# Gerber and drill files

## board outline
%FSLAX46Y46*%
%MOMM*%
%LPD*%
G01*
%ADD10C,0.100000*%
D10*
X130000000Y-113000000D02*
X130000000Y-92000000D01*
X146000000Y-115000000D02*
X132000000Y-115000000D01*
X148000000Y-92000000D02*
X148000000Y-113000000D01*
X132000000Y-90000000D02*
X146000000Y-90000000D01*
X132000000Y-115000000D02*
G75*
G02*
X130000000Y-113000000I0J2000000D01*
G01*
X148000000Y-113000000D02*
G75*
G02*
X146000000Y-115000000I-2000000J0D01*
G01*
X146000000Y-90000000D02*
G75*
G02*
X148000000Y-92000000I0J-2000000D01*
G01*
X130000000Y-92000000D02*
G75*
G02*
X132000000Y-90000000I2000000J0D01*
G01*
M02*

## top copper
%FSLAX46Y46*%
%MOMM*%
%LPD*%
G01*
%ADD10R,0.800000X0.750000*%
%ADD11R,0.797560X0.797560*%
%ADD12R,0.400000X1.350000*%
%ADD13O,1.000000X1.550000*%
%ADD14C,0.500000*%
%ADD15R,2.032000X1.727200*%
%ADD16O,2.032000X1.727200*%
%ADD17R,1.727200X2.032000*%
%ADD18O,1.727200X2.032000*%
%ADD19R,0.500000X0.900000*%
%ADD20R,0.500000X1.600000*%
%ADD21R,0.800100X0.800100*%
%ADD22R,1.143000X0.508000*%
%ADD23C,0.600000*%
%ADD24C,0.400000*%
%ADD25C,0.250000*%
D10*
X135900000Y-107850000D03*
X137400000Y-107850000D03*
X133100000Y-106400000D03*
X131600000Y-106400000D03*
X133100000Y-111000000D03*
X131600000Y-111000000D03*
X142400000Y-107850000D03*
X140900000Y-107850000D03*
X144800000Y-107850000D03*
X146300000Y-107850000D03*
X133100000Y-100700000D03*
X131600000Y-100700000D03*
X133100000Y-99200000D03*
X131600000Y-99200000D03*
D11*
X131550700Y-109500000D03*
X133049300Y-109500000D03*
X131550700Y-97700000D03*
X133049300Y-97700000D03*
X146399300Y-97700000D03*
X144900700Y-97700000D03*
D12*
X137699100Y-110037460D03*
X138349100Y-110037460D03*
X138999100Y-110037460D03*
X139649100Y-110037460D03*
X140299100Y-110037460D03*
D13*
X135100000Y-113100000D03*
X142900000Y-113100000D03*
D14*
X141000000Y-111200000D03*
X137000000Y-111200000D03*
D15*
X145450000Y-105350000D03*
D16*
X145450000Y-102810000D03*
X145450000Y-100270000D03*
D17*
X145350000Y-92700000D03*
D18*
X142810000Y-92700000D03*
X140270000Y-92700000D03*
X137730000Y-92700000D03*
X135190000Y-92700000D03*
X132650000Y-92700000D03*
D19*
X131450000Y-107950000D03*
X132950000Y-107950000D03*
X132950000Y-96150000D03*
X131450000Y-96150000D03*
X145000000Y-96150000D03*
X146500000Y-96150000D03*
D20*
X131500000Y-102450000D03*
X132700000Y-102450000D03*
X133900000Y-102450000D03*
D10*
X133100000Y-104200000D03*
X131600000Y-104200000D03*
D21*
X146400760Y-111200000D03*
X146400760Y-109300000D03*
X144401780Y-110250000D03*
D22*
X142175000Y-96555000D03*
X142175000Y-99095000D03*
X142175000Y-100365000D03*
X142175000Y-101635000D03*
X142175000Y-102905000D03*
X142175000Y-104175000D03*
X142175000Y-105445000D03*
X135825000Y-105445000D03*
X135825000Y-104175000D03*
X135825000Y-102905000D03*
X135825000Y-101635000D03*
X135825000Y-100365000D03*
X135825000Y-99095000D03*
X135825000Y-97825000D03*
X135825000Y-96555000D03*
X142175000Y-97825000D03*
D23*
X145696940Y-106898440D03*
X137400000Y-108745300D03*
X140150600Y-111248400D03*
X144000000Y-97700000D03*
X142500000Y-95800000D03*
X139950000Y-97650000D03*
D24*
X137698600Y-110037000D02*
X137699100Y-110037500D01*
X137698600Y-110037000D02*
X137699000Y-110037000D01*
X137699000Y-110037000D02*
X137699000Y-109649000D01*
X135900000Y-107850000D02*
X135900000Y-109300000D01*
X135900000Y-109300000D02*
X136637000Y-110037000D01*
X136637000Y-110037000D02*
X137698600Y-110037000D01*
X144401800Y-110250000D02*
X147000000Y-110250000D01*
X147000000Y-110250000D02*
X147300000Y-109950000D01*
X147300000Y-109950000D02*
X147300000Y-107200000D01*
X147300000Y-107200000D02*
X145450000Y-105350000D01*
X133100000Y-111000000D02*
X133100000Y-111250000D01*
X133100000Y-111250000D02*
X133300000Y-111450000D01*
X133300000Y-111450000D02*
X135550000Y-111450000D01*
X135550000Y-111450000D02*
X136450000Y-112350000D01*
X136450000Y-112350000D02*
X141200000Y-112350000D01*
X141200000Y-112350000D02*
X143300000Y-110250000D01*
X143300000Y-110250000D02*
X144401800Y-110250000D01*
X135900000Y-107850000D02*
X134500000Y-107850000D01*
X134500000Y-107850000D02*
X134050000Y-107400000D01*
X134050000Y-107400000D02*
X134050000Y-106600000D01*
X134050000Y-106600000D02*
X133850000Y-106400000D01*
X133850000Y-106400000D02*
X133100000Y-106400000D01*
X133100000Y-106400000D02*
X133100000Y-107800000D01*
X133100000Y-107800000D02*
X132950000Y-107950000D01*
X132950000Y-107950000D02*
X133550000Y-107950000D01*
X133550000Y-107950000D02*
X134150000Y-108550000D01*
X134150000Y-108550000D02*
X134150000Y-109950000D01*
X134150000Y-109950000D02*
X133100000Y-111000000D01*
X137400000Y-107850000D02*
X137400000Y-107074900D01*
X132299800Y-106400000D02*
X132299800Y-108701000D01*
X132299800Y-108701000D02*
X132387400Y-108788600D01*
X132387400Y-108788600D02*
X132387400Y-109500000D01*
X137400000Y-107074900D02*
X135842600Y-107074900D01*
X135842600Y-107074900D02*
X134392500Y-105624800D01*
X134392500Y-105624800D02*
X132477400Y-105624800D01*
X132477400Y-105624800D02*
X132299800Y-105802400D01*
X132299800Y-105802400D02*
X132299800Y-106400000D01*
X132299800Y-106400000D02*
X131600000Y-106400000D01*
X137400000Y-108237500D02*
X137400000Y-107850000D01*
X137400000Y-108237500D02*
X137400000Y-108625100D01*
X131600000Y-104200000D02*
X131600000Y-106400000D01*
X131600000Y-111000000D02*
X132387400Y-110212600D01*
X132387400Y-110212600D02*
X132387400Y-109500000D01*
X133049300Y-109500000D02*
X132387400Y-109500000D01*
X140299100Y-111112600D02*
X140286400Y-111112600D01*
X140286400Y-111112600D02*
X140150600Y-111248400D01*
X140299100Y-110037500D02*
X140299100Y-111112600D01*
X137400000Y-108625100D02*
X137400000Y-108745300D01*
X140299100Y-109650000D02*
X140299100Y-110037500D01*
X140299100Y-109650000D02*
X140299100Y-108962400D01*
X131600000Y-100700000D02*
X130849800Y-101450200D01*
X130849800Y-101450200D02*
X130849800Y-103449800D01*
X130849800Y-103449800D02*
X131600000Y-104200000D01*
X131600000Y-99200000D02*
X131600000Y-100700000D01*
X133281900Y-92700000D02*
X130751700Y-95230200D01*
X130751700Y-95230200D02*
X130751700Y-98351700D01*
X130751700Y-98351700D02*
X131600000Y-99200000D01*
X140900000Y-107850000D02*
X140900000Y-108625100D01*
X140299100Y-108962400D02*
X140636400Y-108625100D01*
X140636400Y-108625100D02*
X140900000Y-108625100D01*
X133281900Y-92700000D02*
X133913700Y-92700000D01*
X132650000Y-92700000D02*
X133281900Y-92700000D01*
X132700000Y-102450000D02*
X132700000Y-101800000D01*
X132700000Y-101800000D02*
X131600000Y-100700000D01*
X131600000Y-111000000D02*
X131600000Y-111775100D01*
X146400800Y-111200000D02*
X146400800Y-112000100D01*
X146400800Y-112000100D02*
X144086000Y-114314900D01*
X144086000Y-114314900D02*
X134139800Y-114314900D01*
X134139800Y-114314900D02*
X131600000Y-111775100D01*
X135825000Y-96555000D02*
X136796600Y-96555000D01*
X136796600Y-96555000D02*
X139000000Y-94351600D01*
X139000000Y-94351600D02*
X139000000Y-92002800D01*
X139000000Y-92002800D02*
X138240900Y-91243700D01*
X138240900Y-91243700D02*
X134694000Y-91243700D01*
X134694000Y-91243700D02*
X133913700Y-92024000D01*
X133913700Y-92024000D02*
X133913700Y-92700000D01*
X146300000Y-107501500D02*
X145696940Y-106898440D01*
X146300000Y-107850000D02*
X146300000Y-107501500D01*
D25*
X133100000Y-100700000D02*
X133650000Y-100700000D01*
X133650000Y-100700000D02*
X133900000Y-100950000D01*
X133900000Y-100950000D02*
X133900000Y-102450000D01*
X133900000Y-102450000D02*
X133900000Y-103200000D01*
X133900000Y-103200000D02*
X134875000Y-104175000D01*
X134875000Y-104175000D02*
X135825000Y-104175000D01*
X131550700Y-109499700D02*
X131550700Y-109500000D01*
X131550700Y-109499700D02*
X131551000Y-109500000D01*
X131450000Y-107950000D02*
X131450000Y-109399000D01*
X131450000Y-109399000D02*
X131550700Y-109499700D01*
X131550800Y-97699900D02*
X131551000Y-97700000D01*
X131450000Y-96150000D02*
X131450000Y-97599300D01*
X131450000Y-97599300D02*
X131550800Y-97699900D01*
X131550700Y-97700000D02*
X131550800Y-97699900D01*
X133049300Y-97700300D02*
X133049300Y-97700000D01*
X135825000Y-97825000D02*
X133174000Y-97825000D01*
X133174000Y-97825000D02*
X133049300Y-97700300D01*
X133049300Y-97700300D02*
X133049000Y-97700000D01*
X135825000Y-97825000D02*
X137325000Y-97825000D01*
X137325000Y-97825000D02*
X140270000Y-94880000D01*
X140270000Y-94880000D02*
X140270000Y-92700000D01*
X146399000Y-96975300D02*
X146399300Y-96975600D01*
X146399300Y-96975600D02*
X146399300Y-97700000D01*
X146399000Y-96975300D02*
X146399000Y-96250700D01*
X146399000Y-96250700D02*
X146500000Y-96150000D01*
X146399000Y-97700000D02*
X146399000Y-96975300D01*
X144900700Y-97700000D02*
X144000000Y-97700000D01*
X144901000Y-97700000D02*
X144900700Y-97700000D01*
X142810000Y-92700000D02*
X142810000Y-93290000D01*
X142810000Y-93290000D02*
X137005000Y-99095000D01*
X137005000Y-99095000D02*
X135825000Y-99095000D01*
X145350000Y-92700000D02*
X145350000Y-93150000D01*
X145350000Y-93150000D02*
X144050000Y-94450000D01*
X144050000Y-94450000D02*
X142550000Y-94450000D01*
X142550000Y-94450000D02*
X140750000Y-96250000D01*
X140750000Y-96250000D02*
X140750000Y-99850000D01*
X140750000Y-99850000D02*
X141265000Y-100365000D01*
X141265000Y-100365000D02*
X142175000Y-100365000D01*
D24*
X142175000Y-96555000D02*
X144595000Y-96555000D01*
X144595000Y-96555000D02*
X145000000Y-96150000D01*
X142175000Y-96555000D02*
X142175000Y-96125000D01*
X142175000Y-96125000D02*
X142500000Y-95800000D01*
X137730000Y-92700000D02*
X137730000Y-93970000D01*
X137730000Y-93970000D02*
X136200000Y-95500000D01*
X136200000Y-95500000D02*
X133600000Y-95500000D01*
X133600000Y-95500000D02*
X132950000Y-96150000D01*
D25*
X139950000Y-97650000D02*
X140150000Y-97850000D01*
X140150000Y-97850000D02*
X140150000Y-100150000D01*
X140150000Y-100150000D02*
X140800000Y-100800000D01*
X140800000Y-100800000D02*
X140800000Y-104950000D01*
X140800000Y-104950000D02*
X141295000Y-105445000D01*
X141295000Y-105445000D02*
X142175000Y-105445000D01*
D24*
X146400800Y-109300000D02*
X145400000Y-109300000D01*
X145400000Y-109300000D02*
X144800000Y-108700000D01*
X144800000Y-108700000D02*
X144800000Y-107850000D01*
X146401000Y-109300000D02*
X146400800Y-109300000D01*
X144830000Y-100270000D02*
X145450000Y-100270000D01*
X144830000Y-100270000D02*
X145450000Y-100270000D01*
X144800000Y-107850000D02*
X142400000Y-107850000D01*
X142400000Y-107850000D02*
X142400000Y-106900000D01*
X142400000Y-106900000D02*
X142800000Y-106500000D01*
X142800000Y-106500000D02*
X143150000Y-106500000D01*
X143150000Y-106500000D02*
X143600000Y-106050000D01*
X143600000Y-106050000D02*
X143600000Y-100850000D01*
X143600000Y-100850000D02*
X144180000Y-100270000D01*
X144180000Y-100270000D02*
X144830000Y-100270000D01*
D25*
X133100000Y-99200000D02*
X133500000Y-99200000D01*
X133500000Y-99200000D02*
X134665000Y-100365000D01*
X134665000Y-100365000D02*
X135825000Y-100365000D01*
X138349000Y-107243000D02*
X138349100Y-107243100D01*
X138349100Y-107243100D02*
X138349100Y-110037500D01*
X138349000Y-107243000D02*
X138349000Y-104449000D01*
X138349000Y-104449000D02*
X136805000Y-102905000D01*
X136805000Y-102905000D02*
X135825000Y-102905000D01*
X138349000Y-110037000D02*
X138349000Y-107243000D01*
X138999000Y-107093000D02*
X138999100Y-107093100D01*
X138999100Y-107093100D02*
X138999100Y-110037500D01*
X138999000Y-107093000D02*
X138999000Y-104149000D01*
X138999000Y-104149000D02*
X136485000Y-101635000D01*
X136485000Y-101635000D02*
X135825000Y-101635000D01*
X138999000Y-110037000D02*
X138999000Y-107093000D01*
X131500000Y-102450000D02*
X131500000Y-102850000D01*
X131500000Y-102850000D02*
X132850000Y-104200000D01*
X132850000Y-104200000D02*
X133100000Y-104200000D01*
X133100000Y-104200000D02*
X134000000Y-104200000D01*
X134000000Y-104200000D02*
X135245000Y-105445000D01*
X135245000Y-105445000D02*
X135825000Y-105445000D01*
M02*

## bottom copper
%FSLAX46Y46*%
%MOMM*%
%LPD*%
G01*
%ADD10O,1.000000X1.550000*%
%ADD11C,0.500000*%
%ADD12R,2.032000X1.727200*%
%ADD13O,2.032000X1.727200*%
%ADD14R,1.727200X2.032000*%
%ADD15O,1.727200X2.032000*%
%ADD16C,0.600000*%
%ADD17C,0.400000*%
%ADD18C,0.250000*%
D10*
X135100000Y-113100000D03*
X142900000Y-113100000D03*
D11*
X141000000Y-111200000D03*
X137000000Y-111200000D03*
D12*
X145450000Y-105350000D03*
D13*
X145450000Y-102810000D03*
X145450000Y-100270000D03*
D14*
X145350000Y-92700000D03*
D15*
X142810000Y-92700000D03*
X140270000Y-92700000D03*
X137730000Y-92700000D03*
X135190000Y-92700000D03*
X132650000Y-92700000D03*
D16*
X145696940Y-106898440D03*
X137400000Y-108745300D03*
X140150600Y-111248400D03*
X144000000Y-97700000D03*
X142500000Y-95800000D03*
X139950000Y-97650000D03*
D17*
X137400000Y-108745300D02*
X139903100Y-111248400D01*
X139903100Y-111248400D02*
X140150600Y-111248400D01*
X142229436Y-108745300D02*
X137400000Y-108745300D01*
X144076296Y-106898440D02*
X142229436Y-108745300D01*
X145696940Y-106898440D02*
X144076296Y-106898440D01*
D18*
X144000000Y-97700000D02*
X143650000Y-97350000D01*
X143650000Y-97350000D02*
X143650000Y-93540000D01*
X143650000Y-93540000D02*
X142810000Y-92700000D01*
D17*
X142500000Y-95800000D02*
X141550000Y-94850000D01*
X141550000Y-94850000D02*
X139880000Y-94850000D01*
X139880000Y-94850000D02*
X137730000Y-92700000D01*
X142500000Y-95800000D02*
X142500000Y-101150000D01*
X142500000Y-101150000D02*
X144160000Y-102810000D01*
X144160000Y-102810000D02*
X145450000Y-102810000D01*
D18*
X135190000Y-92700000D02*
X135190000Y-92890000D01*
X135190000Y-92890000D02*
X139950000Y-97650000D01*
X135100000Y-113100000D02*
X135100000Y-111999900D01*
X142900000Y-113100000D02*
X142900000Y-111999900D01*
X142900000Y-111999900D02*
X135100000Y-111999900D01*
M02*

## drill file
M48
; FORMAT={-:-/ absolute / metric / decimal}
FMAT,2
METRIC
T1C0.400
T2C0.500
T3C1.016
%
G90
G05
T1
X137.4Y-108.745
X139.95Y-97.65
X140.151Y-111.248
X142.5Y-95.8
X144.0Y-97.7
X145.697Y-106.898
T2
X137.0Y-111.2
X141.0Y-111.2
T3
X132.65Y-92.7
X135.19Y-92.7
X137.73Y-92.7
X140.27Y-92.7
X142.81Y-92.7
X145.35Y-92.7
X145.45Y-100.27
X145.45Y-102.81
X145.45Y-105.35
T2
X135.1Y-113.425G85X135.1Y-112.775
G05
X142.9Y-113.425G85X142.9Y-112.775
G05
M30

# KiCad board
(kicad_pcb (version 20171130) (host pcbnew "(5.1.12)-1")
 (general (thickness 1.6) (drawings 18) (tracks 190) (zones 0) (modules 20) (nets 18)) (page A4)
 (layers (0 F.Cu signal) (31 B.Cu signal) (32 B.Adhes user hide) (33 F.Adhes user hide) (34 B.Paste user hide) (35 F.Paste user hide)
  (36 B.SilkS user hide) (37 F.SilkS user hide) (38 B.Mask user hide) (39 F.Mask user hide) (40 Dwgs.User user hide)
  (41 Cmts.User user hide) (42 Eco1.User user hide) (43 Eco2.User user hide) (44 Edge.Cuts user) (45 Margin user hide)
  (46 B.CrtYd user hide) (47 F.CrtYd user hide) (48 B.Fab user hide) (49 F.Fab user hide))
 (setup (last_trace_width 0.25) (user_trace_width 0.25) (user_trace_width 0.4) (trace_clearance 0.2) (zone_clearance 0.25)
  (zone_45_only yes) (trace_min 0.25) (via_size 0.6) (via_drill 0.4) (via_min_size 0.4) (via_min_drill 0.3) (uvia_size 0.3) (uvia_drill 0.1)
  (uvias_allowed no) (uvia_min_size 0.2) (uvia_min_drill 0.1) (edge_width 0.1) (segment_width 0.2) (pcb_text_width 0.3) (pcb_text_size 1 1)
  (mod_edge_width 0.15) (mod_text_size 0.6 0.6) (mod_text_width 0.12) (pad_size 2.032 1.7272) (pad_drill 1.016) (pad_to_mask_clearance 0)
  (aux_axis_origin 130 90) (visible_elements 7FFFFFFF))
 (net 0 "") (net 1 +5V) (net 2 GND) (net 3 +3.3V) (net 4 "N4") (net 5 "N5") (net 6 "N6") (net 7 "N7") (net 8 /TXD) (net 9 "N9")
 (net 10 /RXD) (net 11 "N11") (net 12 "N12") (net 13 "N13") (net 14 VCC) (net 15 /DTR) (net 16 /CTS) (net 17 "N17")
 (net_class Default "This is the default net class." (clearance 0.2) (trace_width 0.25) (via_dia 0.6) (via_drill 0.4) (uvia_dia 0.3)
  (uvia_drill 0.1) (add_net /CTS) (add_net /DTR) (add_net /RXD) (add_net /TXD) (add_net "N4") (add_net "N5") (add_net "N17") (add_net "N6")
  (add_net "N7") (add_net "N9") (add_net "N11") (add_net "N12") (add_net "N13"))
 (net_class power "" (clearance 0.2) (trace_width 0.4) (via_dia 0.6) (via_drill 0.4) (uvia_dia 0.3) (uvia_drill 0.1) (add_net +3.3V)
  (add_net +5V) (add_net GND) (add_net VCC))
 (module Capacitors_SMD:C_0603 (layer F.Cu) (at 136.65 107.85)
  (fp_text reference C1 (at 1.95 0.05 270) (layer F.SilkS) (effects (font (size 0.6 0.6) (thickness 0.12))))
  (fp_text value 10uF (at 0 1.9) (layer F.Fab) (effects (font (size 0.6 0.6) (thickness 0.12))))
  (pad 1 smd rect (at -0.75 0) (size 0.8 0.75) (layers F.Cu F.Paste F.Mask) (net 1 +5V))
  (pad 2 smd rect (at 0.75 0) (size 0.8 0.75) (layers F.Cu F.Paste F.Mask) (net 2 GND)))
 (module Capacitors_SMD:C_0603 (layer F.Cu) (at 132.35 106.4 180)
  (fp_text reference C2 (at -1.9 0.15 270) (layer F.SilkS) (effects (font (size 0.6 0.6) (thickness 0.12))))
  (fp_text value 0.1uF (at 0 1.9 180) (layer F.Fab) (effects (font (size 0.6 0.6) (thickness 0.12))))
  (pad 1 smd rect (at -0.75 0 180) (size 0.8 0.75) (layers F.Cu F.Paste F.Mask) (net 1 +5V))
  (pad 2 smd rect (at 0.75 0 180) (size 0.8 0.75) (layers F.Cu F.Paste F.Mask) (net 2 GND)))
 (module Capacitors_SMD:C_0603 (layer F.Cu) (at 132.35 111 180)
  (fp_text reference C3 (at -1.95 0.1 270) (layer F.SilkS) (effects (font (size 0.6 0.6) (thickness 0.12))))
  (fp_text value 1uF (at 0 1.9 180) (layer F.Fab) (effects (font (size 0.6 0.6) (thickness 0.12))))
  (pad 1 smd rect (at -0.75 0 180) (size 0.8 0.75) (layers F.Cu F.Paste F.Mask) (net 1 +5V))
  (pad 2 smd rect (at 0.75 0 180) (size 0.8 0.75) (layers F.Cu F.Paste F.Mask) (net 2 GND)))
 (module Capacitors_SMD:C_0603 (layer F.Cu) (at 141.65 107.85 180)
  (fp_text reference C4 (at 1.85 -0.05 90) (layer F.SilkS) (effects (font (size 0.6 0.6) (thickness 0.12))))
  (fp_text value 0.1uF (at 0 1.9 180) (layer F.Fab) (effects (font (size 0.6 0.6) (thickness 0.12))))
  (pad 1 smd rect (at -0.75 0 180) (size 0.8 0.75) (layers F.Cu F.Paste F.Mask) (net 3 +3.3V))
  (pad 2 smd rect (at 0.75 0 180) (size 0.8 0.75) (layers F.Cu F.Paste F.Mask) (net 2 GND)))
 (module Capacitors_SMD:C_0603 (layer F.Cu) (at 145.55 107.85)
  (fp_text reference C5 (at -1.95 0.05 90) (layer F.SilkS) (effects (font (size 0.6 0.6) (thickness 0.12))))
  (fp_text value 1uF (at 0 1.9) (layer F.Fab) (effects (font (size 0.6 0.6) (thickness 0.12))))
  (pad 1 smd rect (at -0.75 0) (size 0.8 0.75) (layers F.Cu F.Paste F.Mask) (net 3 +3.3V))
  (pad 2 smd rect (at 0.75 0) (size 0.8 0.75) (layers F.Cu F.Paste F.Mask) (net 2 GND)))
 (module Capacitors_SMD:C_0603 (layer F.Cu) (at 132.35 100.7 180)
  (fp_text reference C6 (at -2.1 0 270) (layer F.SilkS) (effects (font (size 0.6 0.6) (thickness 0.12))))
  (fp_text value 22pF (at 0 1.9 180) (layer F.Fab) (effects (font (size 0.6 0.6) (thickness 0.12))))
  (pad 1 smd rect (at -0.75 0 180) (size 0.8 0.75) (layers F.Cu F.Paste F.Mask) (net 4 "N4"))
  (pad 2 smd rect (at 0.75 0 180) (size 0.8 0.75) (layers F.Cu F.Paste F.Mask) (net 2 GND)))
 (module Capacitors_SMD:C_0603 (layer F.Cu) (at 132.35 99.2 180)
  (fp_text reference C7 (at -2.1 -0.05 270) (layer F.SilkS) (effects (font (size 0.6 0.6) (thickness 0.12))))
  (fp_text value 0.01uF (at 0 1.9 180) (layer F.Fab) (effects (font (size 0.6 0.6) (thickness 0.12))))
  (pad 1 smd rect (at -0.75 0 180) (size 0.8 0.75) (layers F.Cu F.Paste F.Mask) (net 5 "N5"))
  (pad 2 smd rect (at 0.75 0 180) (size 0.8 0.75) (layers F.Cu F.Paste F.Mask) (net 2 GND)))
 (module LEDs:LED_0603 (layer F.Cu) (at 132.3 109.5 180)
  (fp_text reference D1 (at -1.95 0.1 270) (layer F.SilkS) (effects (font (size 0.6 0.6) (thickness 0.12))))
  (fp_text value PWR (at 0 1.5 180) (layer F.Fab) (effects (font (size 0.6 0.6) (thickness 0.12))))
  (pad 2 smd rect (at 0.7493 0) (size 0.79756 0.79756) (layers F.Cu F.Paste F.Mask) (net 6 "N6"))
  (pad 1 smd rect (at -0.7493 0) (size 0.79756 0.79756) (layers F.Cu F.Paste F.Mask) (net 2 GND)))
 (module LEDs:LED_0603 (layer F.Cu) (at 132.3 97.7 180)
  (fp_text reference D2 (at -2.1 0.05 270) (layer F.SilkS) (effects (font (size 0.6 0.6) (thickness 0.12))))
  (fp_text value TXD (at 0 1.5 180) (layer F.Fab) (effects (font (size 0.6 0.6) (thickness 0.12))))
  (pad 2 smd rect (at 0.7493 0) (size 0.79756 0.79756) (layers F.Cu F.Paste F.Mask) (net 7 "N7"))
  (pad 1 smd rect (at -0.7493 0) (size 0.79756 0.79756) (layers F.Cu F.Paste F.Mask) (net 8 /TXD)))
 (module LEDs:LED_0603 (layer F.Cu) (at 145.65 97.7)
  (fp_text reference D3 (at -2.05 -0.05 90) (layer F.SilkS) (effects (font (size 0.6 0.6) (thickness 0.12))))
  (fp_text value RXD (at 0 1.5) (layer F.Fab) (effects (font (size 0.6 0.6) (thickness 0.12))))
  (pad 2 smd rect (at 0.7493 0 180) (size 0.79756 0.79756) (layers F.Cu F.Paste F.Mask) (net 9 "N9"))
  (pad 1 smd rect (at -0.7493 0 180) (size 0.79756 0.79756) (layers F.Cu F.Paste F.Mask) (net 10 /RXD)))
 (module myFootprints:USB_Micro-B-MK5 (layer F.Cu) (at 139 111.6)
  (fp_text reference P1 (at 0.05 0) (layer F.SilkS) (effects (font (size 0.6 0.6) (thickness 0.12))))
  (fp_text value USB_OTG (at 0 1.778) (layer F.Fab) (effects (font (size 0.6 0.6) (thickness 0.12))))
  (pad 1 smd rect (at -1.3009 -1.56254 90) (size 1.35 0.4) (layers F.Cu F.Paste F.Mask) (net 1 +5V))
  (pad 2 smd rect (at -0.6509 -1.56254 90) (size 1.35 0.4) (layers F.Cu F.Paste F.Mask) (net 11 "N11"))
  (pad 3 smd rect (at -0.0009 -1.56254 90) (size 1.35 0.4) (layers F.Cu F.Paste F.Mask) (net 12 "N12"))
  (pad 4 smd rect (at 0.6491 -1.56254 90) (size 1.35 0.4) (layers F.Cu F.Paste F.Mask))
  (pad 5 smd rect (at 1.2991 -1.56254 90) (size 1.35 0.4) (layers F.Cu F.Paste F.Mask) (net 2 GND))
  (pad 6 thru_hole oval (at -3.9 1.5 90) (size 1.55 1) (drill oval 1.15 0.5) (layers *.Cu *.Mask F.SilkS) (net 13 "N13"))
  (pad 6 thru_hole oval (at 3.9 1.5 90) (size 1.55 1) (drill oval 1.15 0.5) (layers *.Cu *.Mask F.SilkS) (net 13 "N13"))
  (pad "" thru_hole circle (at 2 -0.4) (size 0.5 0.5) (drill 0.5) (layers *.Cu *.Mask F.SilkS) (zone_connect 0))
  (pad "" thru_hole circle (at -2 -0.4) (size 0.5 0.5) (drill 0.5) (layers *.Cu *.Mask F.SilkS) (zone_connect 0)))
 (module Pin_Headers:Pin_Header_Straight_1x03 (layer F.Cu) (at 145.45 105.35 180)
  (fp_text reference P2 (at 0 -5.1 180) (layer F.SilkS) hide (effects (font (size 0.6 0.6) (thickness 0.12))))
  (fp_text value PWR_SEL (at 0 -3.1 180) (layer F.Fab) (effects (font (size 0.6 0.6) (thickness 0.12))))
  (pad 1 thru_hole rect (at 0 0 180) (size 2.032 1.7272) (drill 1.016) (layers *.Cu *.Mask F.SilkS) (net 1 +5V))
  (pad 2 thru_hole oval (at 0 2.54 180) (size 2.032 1.7272) (drill 1.016) (layers *.Cu *.Mask F.SilkS) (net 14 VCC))
  (pad 3 thru_hole oval (at 0 5.08 180) (size 2.032 1.7272) (drill 1.016) (layers *.Cu *.Mask F.SilkS) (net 3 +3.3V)))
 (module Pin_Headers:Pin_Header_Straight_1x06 (layer F.Cu) (at 145.35 92.7 270)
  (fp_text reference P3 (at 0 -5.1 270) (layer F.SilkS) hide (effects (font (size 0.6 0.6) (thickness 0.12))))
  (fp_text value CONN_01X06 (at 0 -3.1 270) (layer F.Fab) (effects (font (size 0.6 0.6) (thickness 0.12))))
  (pad 1 thru_hole rect (at 0 0 270) (size 2.032 1.7272) (drill 1.016) (layers *.Cu *.Mask F.SilkS) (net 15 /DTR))
  (pad 2 thru_hole oval (at 0 2.54 270) (size 2.032 1.7272) (drill 1.016) (layers *.Cu *.Mask F.SilkS) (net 10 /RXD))
  (pad 3 thru_hole oval (at 0 5.08 270) (size 2.032 1.7272) (drill 1.016) (layers *.Cu *.Mask F.SilkS) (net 8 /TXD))
  (pad 4 thru_hole oval (at 0 7.62 270) (size 2.032 1.7272) (drill 1.016) (layers *.Cu *.Mask F.SilkS) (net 14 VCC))
  (pad 5 thru_hole oval (at 0 10.16 270) (size 2.032 1.7272) (drill 1.016) (layers *.Cu *.Mask F.SilkS) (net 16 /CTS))
  (pad 6 thru_hole oval (at 0 12.7 270) (size 2.032 1.7272) (drill 1.016) (layers *.Cu *.Mask F.SilkS) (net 2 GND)))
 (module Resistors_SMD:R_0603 (layer F.Cu) (at 132.2 107.95)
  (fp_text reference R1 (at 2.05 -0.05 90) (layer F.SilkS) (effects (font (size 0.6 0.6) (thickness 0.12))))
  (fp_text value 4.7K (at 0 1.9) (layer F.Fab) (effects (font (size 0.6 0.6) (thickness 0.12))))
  (pad 1 smd rect (at -0.75 0) (size 0.5 0.9) (layers F.Cu F.Paste F.Mask) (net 6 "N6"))
  (pad 2 smd rect (at 0.75 0) (size 0.5 0.9) (layers F.Cu F.Paste F.Mask) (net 1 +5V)))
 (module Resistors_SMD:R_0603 (layer F.Cu) (at 132.2 96.15 180)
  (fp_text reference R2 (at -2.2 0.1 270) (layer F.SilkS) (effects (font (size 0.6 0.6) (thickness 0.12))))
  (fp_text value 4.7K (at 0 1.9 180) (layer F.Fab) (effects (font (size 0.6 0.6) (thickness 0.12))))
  (pad 1 smd rect (at -0.75 0 180) (size 0.5 0.9) (layers F.Cu F.Paste F.Mask) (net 14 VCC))
  (pad 2 smd rect (at 0.75 0 180) (size 0.5 0.9) (layers F.Cu F.Paste F.Mask) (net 7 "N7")))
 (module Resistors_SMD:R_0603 (layer F.Cu) (at 145.75 96.15)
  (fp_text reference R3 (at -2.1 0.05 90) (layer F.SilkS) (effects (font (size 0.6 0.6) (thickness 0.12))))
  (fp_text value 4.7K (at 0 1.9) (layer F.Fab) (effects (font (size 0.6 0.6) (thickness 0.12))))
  (pad 1 smd rect (at -0.75 0) (size 0.5 0.9) (layers F.Cu F.Paste F.Mask) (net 14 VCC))
  (pad 2 smd rect (at 0.75 0) (size 0.5 0.9) (layers F.Cu F.Paste F.Mask) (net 9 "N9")))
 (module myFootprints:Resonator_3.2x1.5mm (layer F.Cu) (at 132.7 102.45 180)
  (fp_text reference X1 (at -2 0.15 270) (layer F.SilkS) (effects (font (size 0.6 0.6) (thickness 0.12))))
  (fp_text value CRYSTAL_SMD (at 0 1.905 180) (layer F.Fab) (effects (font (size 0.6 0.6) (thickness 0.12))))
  (pad 2 smd rect (at 1.2 0 180) (size 0.5 1.6) (layers F.Cu F.Paste F.Mask) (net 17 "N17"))
  (pad 3 smd rect (at 0 0 180) (size 0.5 1.6) (layers F.Cu F.Paste F.Mask) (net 2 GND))
  (pad 1 smd rect (at -1.2 0 180) (size 0.5 1.6) (layers F.Cu F.Paste F.Mask) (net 4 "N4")))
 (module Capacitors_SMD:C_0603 (layer F.Cu) (at 132.35 104.2 180)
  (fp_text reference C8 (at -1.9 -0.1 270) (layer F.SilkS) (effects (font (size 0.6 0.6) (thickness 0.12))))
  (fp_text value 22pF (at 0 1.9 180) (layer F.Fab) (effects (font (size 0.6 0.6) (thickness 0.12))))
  (pad 1 smd rect (at -0.75 0 180) (size 0.8 0.75) (layers F.Cu F.Paste F.Mask) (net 17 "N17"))
  (pad 2 smd rect (at 0.75 0 180) (size 0.8 0.75) (layers F.Cu F.Paste F.Mask) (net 2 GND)))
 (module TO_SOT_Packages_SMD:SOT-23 (layer F.Cu) (at 145.4 110.25 90)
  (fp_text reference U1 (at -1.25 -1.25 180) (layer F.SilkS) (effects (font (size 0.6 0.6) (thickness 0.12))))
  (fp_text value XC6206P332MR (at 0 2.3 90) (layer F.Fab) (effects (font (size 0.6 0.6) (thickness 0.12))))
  (pad 1 smd rect (at -0.95 1.00076 90) (size 0.8001 0.8001) (layers F.Cu F.Paste F.Mask) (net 2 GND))
  (pad 2 smd rect (at 0.95 1.00076 90) (size 0.8001 0.8001) (layers F.Cu F.Paste F.Mask) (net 3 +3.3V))
  (pad 3 smd rect (at 0 -0.99822 90) (size 0.8001 0.8001) (layers F.Cu F.Paste F.Mask) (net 1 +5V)))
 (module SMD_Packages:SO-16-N (layer F.Cu) (at 139 101 270)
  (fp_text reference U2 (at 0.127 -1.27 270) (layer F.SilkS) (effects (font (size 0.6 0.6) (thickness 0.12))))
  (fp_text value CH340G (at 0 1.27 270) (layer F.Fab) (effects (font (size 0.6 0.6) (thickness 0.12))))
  (pad 16 smd rect (at -4.445 -3.175 270) (size 0.508 1.143) (layers F.Cu F.Paste F.Mask) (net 14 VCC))
  (pad 14 smd rect (at -1.905 -3.175 270) (size 0.508 1.143) (layers F.Cu F.Paste F.Mask))
  (pad 13 smd rect (at -0.635 -3.175 270) (size 0.508 1.143) (layers F.Cu F.Paste F.Mask) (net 15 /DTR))
  (pad 12 smd rect (at 0.635 -3.175 270) (size 0.508 1.143) (layers F.Cu F.Paste F.Mask))
  (pad 11 smd rect (at 1.905 -3.175 270) (size 0.508 1.143) (layers F.Cu F.Paste F.Mask))
  (pad 10 smd rect (at 3.175 -3.175 270) (size 0.508 1.143) (layers F.Cu F.Paste F.Mask))
  (pad 9 smd rect (at 4.445 -3.175 270) (size 0.508 1.143) (layers F.Cu F.Paste F.Mask) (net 16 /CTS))
  (pad 8 smd rect (at 4.445 3.175 270) (size 0.508 1.143) (layers F.Cu F.Paste F.Mask) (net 17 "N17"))
  (pad 7 smd rect (at 3.175 3.175 270) (size 0.508 1.143) (layers F.Cu F.Paste F.Mask) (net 4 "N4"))
  (pad 6 smd rect (at 1.905 3.175 270) (size 0.508 1.143) (layers F.Cu F.Paste F.Mask) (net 11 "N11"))
  (pad 5 smd rect (at 0.635 3.175 270) (size 0.508 1.143) (layers F.Cu F.Paste F.Mask) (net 12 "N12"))
  (pad 4 smd rect (at -0.635 3.175 270) (size 0.508 1.143) (layers F.Cu F.Paste F.Mask) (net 5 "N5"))
  (pad 3 smd rect (at -1.905 3.175 270) (size 0.508 1.143) (layers F.Cu F.Paste F.Mask) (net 10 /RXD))
  (pad 2 smd rect (at -3.175 3.175 270) (size 0.508 1.143) (layers F.Cu F.Paste F.Mask) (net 8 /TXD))
  (pad 1 smd rect (at -4.445 3.175 270) (size 0.508 1.143) (layers F.Cu F.Paste F.Mask) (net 2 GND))
  (pad 15 smd rect (at -3.175 -3.175 270) (size 0.508 1.143) (layers F.Cu F.Paste F.Mask)))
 (gr_line (start 130 113) (end 130 92) (angle 90) (layer Edge.Cuts) (width 0.1))
 (gr_line (start 146 115) (end 132 115) (angle 90) (layer Edge.Cuts) (width 0.1))
 (gr_line (start 148 92) (end 148 113) (angle 90) (layer Edge.Cuts) (width 0.1))
 (gr_line (start 132 90) (end 146 90) (angle 90) (layer Edge.Cuts) (width 0.1))
 (gr_arc (start 132 113) (end 132 115) (angle 90) (layer Edge.Cuts) (width 0.1))
 (gr_arc (start 146 113) (end 148 113) (angle 90) (layer Edge.Cuts) (width 0.1))
 (gr_arc (start 146 92) (end 146 90) (angle 90) (layer Edge.Cuts) (width 0.1))
 (gr_arc (start 132 92) (end 130 92) (angle 90) (layer Edge.Cuts) (width 0.1))
 (via (at 145.69694 106.89844) (size 0.6) (drill 0.4) (layers F.Cu B.Cu) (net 2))
 (segment (start 137.6986 110.037) (end 137.6991 110.0375) (width 0.4) (layer F.Cu) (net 1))
 (segment (start 137.6986 110.037) (end 137.699 110.037) (width 0.4) (layer F.Cu) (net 1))
 (segment (start 137.699 110.037) (end 137.699 109.649) (width 0.4) (layer F.Cu) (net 1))
 (segment (start 135.9 107.85) (end 135.9 109.3) (width 0.4) (layer F.Cu) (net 1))
 (segment (start 135.9 109.3) (end 136.637 110.037) (width 0.4) (layer F.Cu) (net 1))
 (segment (start 136.637 110.037) (end 137.6986 110.037) (width 0.4) (layer F.Cu) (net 1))
 (segment (start 144.4018 110.25) (end 147 110.25) (width 0.4) (layer F.Cu) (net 1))
 (segment (start 147 110.25) (end 147.3 109.95) (width 0.4) (layer F.Cu) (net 1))
 (segment (start 147.3 109.95) (end 147.3 107.2) (width 0.4) (layer F.Cu) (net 1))
 (segment (start 147.3 107.2) (end 145.45 105.35) (width 0.4) (layer F.Cu) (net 1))
 (segment (start 133.1 111) (end 133.1 111.25) (width 0.4) (layer F.Cu) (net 1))
 (segment (start 133.1 111.25) (end 133.3 111.45) (width 0.4) (layer F.Cu) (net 1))
 (segment (start 133.3 111.45) (end 135.55 111.45) (width 0.4) (layer F.Cu) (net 1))
 (segment (start 135.55 111.45) (end 136.45 112.35) (width 0.4) (layer F.Cu) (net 1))
 (segment (start 136.45 112.35) (end 141.2 112.35) (width 0.4) (layer F.Cu) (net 1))
 (segment (start 141.2 112.35) (end 143.3 110.25) (width 0.4) (layer F.Cu) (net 1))
 (segment (start 143.3 110.25) (end 144.4018 110.25) (width 0.4) (layer F.Cu) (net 1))
 (segment (start 135.9 107.85) (end 134.5 107.85) (width 0.4) (layer F.Cu) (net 1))
 (segment (start 134.5 107.85) (end 134.05 107.4) (width 0.4) (layer F.Cu) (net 1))
 (segment (start 134.05 107.4) (end 134.05 106.6) (width 0.4) (layer F.Cu) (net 1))
 (segment (start 134.05 106.6) (end 133.85 106.4) (width 0.4) (layer F.Cu) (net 1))
 (segment (start 133.85 106.4) (end 133.1 106.4) (width 0.4) (layer F.Cu) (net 1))
 (segment (start 133.1 106.4) (end 133.1 107.8) (width 0.4) (layer F.Cu) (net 1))
 (segment (start 133.1 107.8) (end 132.95 107.95) (width 0.4) (layer F.Cu) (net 1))
 (segment (start 132.95 107.95) (end 133.55 107.95) (width 0.4) (layer F.Cu) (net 1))
 (segment (start 133.55 107.95) (end 134.15 108.55) (width 0.4) (layer F.Cu) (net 1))
 (segment (start 134.15 108.55) (end 134.15 109.95) (width 0.4) (layer F.Cu) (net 1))
 (segment (start 134.15 109.95) (end 133.1 111) (width 0.4) (layer F.Cu) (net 1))
 (segment (start 137.4 107.85) (end 137.4 107.0749) (width 0.4) (layer F.Cu) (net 2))
 (segment (start 132.2998 106.4) (end 132.2998 108.701) (width 0.4) (layer F.Cu) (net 2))
 (segment (start 132.2998 108.701) (end 132.3874 108.7886) (width 0.4) (layer F.Cu) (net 2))
 (segment (start 132.3874 108.7886) (end 132.3874 109.5) (width 0.4) (layer F.Cu) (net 2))
 (segment (start 137.4 107.0749) (end 135.8426 107.0749) (width 0.4) (layer F.Cu) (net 2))
 (segment (start 135.8426 107.0749) (end 134.3925 105.6248) (width 0.4) (layer F.Cu) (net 2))
 (segment (start 134.3925 105.6248) (end 132.4774 105.6248) (width 0.4) (layer F.Cu) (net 2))
 (segment (start 132.4774 105.6248) (end 132.2998 105.8024) (width 0.4) (layer F.Cu) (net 2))
 (segment (start 132.2998 105.8024) (end 132.2998 106.4) (width 0.4) (layer F.Cu) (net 2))
 (segment (start 132.2998 106.4) (end 131.6 106.4) (width 0.4) (layer F.Cu) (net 2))
 (segment (start 137.4 108.2375) (end 137.4 107.85) (width 0.4) (layer F.Cu) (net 2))
 (segment (start 137.4 108.2375) (end 137.4 108.6251) (width 0.4) (layer F.Cu) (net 2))
 (segment (start 131.6 104.2) (end 131.6 106.4) (width 0.4) (layer F.Cu) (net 2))
 (segment (start 131.6 111) (end 132.3874 110.2126) (width 0.4) (layer F.Cu) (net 2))
 (segment (start 132.3874 110.2126) (end 132.3874 109.5) (width 0.4) (layer F.Cu) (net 2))
 (segment (start 133.0493 109.5) (end 132.3874 109.5) (width 0.4) (layer F.Cu) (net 2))
 (segment (start 140.2991 111.1126) (end 140.2864 111.1126) (width 0.4) (layer F.Cu) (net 2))
 (segment (start 140.2864 111.1126) (end 140.1506 111.2484) (width 0.4) (layer F.Cu) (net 2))
 (segment (start 137.4 108.7453) (end 139.9031 111.2484) (width 0.4) (layer B.Cu) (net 2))
 (segment (start 139.9031 111.2484) (end 140.1506 111.2484) (width 0.4) (layer B.Cu) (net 2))
 (segment (start 140.2991 110.0375) (end 140.2991 111.1126) (width 0.4) (layer F.Cu) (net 2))
 (segment (start 137.4 108.6251) (end 137.4 108.7453) (width 0.4) (layer F.Cu) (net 2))
 (segment (start 140.2991 109.65) (end 140.2991 110.0375) (width 0.4) (layer F.Cu) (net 2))
 (segment (start 140.2991 109.65) (end 140.2991 108.9624) (width 0.4) (layer F.Cu) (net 2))
 (segment (start 131.6 100.7) (end 130.8498 101.4502) (width 0.4) (layer F.Cu) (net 2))
 (segment (start 130.8498 101.4502) (end 130.8498 103.4498) (width 0.4) (layer F.Cu) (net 2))
 (segment (start 130.8498 103.4498) (end 131.6 104.2) (width 0.4) (layer F.Cu) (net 2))
 (segment (start 131.6 99.2) (end 131.6 100.7) (width 0.4) (layer F.Cu) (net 2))
 (segment (start 133.2819 92.7) (end 130.7517 95.2302) (width 0.4) (layer F.Cu) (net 2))
 (segment (start 130.7517 95.2302) (end 130.7517 98.3517) (width 0.4) (layer F.Cu) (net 2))
 (segment (start 130.7517 98.3517) (end 131.6 99.2) (width 0.4) (layer F.Cu) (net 2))
 (segment (start 140.9 107.85) (end 140.9 108.6251) (width 0.4) (layer F.Cu) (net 2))
 (segment (start 140.2991 108.9624) (end 140.6364 108.6251) (width 0.4) (layer F.Cu) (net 2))
 (segment (start 140.6364 108.6251) (end 140.9 108.6251) (width 0.4) (layer F.Cu) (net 2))
 (segment (start 133.2819 92.7) (end 133.9137 92.7) (width 0.4) (layer F.Cu) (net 2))
 (segment (start 132.65 92.7) (end 133.2819 92.7) (width 0.4) (layer F.Cu) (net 2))
 (segment (start 132.7 102.45) (end 132.7 101.8) (width 0.4) (layer F.Cu) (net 2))
 (segment (start 132.7 101.8) (end 131.6 100.7) (width 0.4) (layer F.Cu) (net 2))
 (segment (start 131.6 111) (end 131.6 111.7751) (width 0.4) (layer F.Cu) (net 2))
 (segment (start 146.4008 111.2) (end 146.4008 112.0001) (width 0.4) (layer F.Cu) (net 2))
 (segment (start 146.4008 112.0001) (end 144.086 114.3149) (width 0.4) (layer F.Cu) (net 2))
 (segment (start 144.086 114.3149) (end 134.1398 114.3149) (width 0.4) (layer F.Cu) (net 2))
 (segment (start 134.1398 114.3149) (end 131.6 111.7751) (width 0.4) (layer F.Cu) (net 2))
 (segment (start 135.825 96.555) (end 136.7966 96.555) (width 0.4) (layer F.Cu) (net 2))
 (segment (start 136.7966 96.555) (end 139 94.3516) (width 0.4) (layer F.Cu) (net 2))
 (segment (start 139 94.3516) (end 139 92.0028) (width 0.4) (layer F.Cu) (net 2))
 (segment (start 139 92.0028) (end 138.2409 91.2437) (width 0.4) (layer F.Cu) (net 2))
 (segment (start 138.2409 91.2437) (end 134.694 91.2437) (width 0.4) (layer F.Cu) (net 2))
 (segment (start 134.694 91.2437) (end 133.9137 92.024) (width 0.4) (layer F.Cu) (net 2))
 (segment (start 133.9137 92.024) (end 133.9137 92.7) (width 0.4) (layer F.Cu) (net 2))
 (via (at 137.4 108.7453) (size 0.6) (layers F.Cu B.Cu) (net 2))
 (via (at 140.1506 111.2484) (size 0.6) (layers F.Cu B.Cu) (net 2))
 (segment (start 146.3 107.5015) (end 145.69694 106.89844) (width 0.4) (layer F.Cu) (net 2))
 (segment (start 146.3 107.85) (end 146.3 107.5015) (width 0.4) (layer F.Cu) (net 2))
 (segment (start 142.229436 108.7453) (end 137.4 108.7453) (width 0.4) (layer B.Cu) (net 2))
 (segment (start 144.076296 106.89844) (end 142.229436 108.7453) (width 0.4) (layer B.Cu) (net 2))
 (segment (start 145.69694 106.89844) (end 144.076296 106.89844) (width 0.4) (layer B.Cu) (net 2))
 (segment (start 133.1 100.7) (end 133.65 100.7) (width 0.25) (layer F.Cu) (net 4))
 (segment (start 133.65 100.7) (end 133.9 100.95) (width 0.25) (layer F.Cu) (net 4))
 (segment (start 133.9 100.95) (end 133.9 102.45) (width 0.25) (layer F.Cu) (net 4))
 (segment (start 133.9 102.45) (end 133.9 103.2) (width 0.25) (layer F.Cu) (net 4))
 (segment (start 133.9 103.2) (end 134.875 104.175) (width 0.25) (layer F.Cu) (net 4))
 (segment (start 134.875 104.175) (end 135.825 104.175) (width 0.25) (layer F.Cu) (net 4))
 (segment (start 131.5507 109.4997) (end 131.5507 109.5) (width 0.25) (layer F.Cu) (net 6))
 (segment (start 131.5507 109.4997) (end 131.551 109.5) (width 0.25) (layer F.Cu) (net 6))
 (segment (start 131.45 107.95) (end 131.45 109.399) (width 0.25) (layer F.Cu) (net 6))
 (segment (start 131.45 109.399) (end 131.5507 109.4997) (width 0.25) (layer F.Cu) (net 6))
 (segment (start 131.5508 97.6999) (end 131.551 97.7) (width 0.25) (layer F.Cu) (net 7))
 (segment (start 131.45 96.15) (end 131.45 97.5993) (width 0.25) (layer F.Cu) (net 7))
 (segment (start 131.45 97.5993) (end 131.5508 97.6999) (width 0.25) (layer F.Cu) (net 7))
 (segment (start 131.5507 97.7) (end 131.5508 97.6999) (width 0.25) (layer F.Cu) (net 7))
 (segment (start 133.0493 97.7003) (end 133.0493 97.7) (width 0.25) (layer F.Cu) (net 8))
 (segment (start 135.825 97.825) (end 133.174 97.825) (width 0.25) (layer F.Cu) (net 8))
 (segment (start 133.174 97.825) (end 133.0493 97.7003) (width 0.25) (layer F.Cu) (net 8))
 (segment (start 133.0493 97.7003) (end 133.049 97.7) (width 0.25) (layer F.Cu) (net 8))
 (segment (start 135.825 97.825) (end 137.325 97.825) (width 0.25) (layer F.Cu) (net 8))
 (segment (start 137.325 97.825) (end 140.27 94.88) (width 0.25) (layer F.Cu) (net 8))
 (segment (start 140.27 94.88) (end 140.27 92.7) (width 0.25) (layer F.Cu) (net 8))
 (segment (start 146.399 96.9753) (end 146.3993 96.9756) (width 0.25) (layer F.Cu) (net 9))
 (segment (start 146.3993 96.9756) (end 146.3993 97.7) (width 0.25) (layer F.Cu) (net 9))
 (segment (start 146.399 96.9753) (end 146.399 96.2507) (width 0.25) (layer F.Cu) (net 9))
 (segment (start 146.399 96.2507) (end 146.5 96.15) (width 0.25) (layer F.Cu) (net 9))
 (segment (start 146.399 97.7) (end 146.399 96.9753) (width 0.25) (layer F.Cu) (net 9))
 (segment (start 144.9007 97.7) (end 144 97.7) (width 0.25) (layer F.Cu) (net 10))
 (segment (start 144.901 97.7) (end 144.9007 97.7) (width 0.25) (layer F.Cu) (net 10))
 (segment (start 142.81 92.7) (end 142.81 93.29) (width 0.25) (layer F.Cu) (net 10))
 (segment (start 142.81 93.29) (end 137.005 99.095) (width 0.25) (layer F.Cu) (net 10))
 (segment (start 137.005 99.095) (end 135.825 99.095) (width 0.25) (layer F.Cu) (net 10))
 (segment (start 144 97.7) (end 143.65 97.35) (width 0.25) (layer B.Cu) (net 10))
 (segment (start 143.65 97.35) (end 143.65 93.54) (width 0.25) (layer B.Cu) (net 10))
 (segment (start 143.65 93.54) (end 142.81 92.7) (width 0.25) (layer B.Cu) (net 10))
 (via (at 144 97.7) (size 0.6) (layers F.Cu B.Cu) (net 10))
 (segment (start 145.35 92.7) (end 145.35 93.15) (width 0.25) (layer F.Cu) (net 15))
 (segment (start 145.35 93.15) (end 144.05 94.45) (width 0.25) (layer F.Cu) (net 15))
 (segment (start 144.05 94.45) (end 142.55 94.45) (width 0.25) (layer F.Cu) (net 15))
 (segment (start 142.55 94.45) (end 140.75 96.25) (width 0.25) (layer F.Cu) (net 15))
 (segment (start 140.75 96.25) (end 140.75 99.85) (width 0.25) (layer F.Cu) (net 15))
 (segment (start 140.75 99.85) (end 141.265 100.365) (width 0.25) (layer F.Cu) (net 15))
 (segment (start 141.265 100.365) (end 142.175 100.365) (width 0.25) (layer F.Cu) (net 15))
 (segment (start 142.175 96.555) (end 144.595 96.555) (width 0.4) (layer F.Cu) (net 14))
 (segment (start 144.595 96.555) (end 145 96.15) (width 0.4) (layer F.Cu) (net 14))
 (segment (start 142.175 96.555) (end 142.175 96.125) (width 0.4) (layer F.Cu) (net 14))
 (segment (start 142.175 96.125) (end 142.5 95.8) (width 0.4) (layer F.Cu) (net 14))
 (segment (start 137.73 92.7) (end 137.73 93.97) (width 0.4) (layer F.Cu) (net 14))
 (segment (start 137.73 93.97) (end 136.2 95.5) (width 0.4) (layer F.Cu) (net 14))
 (segment (start 136.2 95.5) (end 133.6 95.5) (width 0.4) (layer F.Cu) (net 14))
 (segment (start 133.6 95.5) (end 132.95 96.15) (width 0.4) (layer F.Cu) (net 14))
 (segment (start 142.5 95.8) (end 141.55 94.85) (width 0.4) (layer B.Cu) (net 14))
 (segment (start 141.55 94.85) (end 139.88 94.85) (width 0.4) (layer B.Cu) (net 14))
 (segment (start 139.88 94.85) (end 137.73 92.7) (width 0.4) (layer B.Cu) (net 14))
 (segment (start 142.5 95.8) (end 142.5 101.15) (width 0.4) (layer B.Cu) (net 14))
 (segment (start 142.5 101.15) (end 144.16 102.81) (width 0.4) (layer B.Cu) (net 14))
 (segment (start 144.16 102.81) (end 145.45 102.81) (width 0.4) (layer B.Cu) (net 14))
 (via (at 142.5 95.8) (size 0.6) (layers F.Cu B.Cu) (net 14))
 (segment (start 139.95 97.65) (end 140.15 97.85) (width 0.25) (layer F.Cu) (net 16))
 (segment (start 140.15 97.85) (end 140.15 100.15) (width 0.25) (layer F.Cu) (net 16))
 (segment (start 140.15 100.15) (end 140.8 100.8) (width 0.25) (layer F.Cu) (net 16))
 (segment (start 140.8 100.8) (end 140.8 104.95) (width 0.25) (layer F.Cu) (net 16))
 (segment (start 140.8 104.95) (end 141.295 105.445) (width 0.25) (layer F.Cu) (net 16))
 (segment (start 141.295 105.445) (end 142.175 105.445) (width 0.25) (layer F.Cu) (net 16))
 (segment (start 135.19 92.7) (end 135.19 92.89) (width 0.25) (layer B.Cu) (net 16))
 (segment (start 135.19 92.89) (end 139.95 97.65) (width 0.25) (layer B.Cu) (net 16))
 (via (at 139.95 97.65) (size 0.6) (layers F.Cu B.Cu) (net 16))
 (segment (start 146.4008 109.3) (end 145.4 109.3) (width 0.4) (layer F.Cu) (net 3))
 (segment (start 145.4 109.3) (end 144.8 108.7) (width 0.4) (layer F.Cu) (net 3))
 (segment (start 144.8 108.7) (end 144.8 107.85) (width 0.4) (layer F.Cu) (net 3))
 (segment (start 146.401 109.3) (end 146.4008 109.3) (width 0.4) (layer F.Cu) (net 3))
 (segment (start 144.83 100.27) (end 145.45 100.27) (width 0.4) (layer F.Cu) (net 3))
 (segment (start 144.83 100.27) (end 145.45 100.27) (width 0.4) (layer F.Cu) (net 3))
 (segment (start 144.8 107.85) (end 142.4 107.85) (width 0.4) (layer F.Cu) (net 3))
 (segment (start 142.4 107.85) (end 142.4 106.9) (width 0.4) (layer F.Cu) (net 3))
 (segment (start 142.4 106.9) (end 142.8 106.5) (width 0.4) (layer F.Cu) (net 3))
 (segment (start 142.8 106.5) (end 143.15 106.5) (width 0.4) (layer F.Cu) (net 3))
 (segment (start 143.15 106.5) (end 143.6 106.05) (width 0.4) (layer F.Cu) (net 3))
 (segment (start 143.6 106.05) (end 143.6 100.85) (width 0.4) (layer F.Cu) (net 3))
 (segment (start 143.6 100.85) (end 144.18 100.27) (width 0.4) (layer F.Cu) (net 3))
 (segment (start 144.18 100.27) (end 144.83 100.27) (width 0.4) (layer F.Cu) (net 3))
 (segment (start 133.1 99.2) (end 133.5 99.2) (width 0.25) (layer F.Cu) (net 5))
 (segment (start 133.5 99.2) (end 134.665 100.365) (width 0.25) (layer F.Cu) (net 5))
 (segment (start 134.665 100.365) (end 135.825 100.365) (width 0.25) (layer F.Cu) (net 5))
 (segment (start 138.349 107.243) (end 138.3491 107.2431) (width 0.25) (layer F.Cu) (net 11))
 (segment (start 138.3491 107.2431) (end 138.3491 110.0375) (width 0.25) (layer F.Cu) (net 11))
 (segment (start 138.349 107.243) (end 138.349 104.449) (width 0.25) (layer F.Cu) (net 11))
 (segment (start 138.349 104.449) (end 136.805 102.905) (width 0.25) (layer F.Cu) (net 11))
 (segment (start 136.805 102.905) (end 135.825 102.905) (width 0.25) (layer F.Cu) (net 11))
 (segment (start 138.349 110.037) (end 138.349 107.243) (width 0.25) (layer F.Cu) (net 11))
 (segment (start 138.999 107.093) (end 138.9991 107.0931) (width 0.25) (layer F.Cu) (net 12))
 (segment (start 138.9991 107.0931) (end 138.9991 110.0375) (width 0.25) (layer F.Cu) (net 12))
 (segment (start 138.999 107.093) (end 138.999 104.149) (width 0.25) (layer F.Cu) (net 12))
 (segment (start 138.999 104.149) (end 136.485 101.635) (width 0.25) (layer F.Cu) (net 12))
 (segment (start 136.485 101.635) (end 135.825 101.635) (width 0.25) (layer F.Cu) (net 12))
 (segment (start 138.999 110.037) (end 138.999 107.093) (width 0.25) (layer F.Cu) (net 12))
 (segment (start 135.1 113.1) (end 135.1 111.9999) (width 0.25) (layer B.Cu) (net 13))
 (segment (start 142.9 113.1) (end 142.9 111.9999) (width 0.25) (layer B.Cu) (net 13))
 (segment (start 142.9 111.9999) (end 135.1 111.9999) (width 0.25) (layer B.Cu) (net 13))
 (segment (start 131.5 102.45) (end 131.5 102.85) (width 0.25) (layer F.Cu) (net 17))
 (segment (start 131.5 102.85) (end 132.85 104.2) (width 0.25) (layer F.Cu) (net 17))
 (segment (start 132.85 104.2) (end 133.1 104.2) (width 0.25) (layer F.Cu) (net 17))
 (segment (start 133.1 104.2) (end 134 104.2) (width 0.25) (layer F.Cu) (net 17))
 (segment (start 134 104.2) (end 135.245 105.445) (width 0.25) (layer F.Cu) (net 17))
 (segment (start 135.245 105.445) (end 135.825 105.445) (width 0.25) (layer F.Cu) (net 17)))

